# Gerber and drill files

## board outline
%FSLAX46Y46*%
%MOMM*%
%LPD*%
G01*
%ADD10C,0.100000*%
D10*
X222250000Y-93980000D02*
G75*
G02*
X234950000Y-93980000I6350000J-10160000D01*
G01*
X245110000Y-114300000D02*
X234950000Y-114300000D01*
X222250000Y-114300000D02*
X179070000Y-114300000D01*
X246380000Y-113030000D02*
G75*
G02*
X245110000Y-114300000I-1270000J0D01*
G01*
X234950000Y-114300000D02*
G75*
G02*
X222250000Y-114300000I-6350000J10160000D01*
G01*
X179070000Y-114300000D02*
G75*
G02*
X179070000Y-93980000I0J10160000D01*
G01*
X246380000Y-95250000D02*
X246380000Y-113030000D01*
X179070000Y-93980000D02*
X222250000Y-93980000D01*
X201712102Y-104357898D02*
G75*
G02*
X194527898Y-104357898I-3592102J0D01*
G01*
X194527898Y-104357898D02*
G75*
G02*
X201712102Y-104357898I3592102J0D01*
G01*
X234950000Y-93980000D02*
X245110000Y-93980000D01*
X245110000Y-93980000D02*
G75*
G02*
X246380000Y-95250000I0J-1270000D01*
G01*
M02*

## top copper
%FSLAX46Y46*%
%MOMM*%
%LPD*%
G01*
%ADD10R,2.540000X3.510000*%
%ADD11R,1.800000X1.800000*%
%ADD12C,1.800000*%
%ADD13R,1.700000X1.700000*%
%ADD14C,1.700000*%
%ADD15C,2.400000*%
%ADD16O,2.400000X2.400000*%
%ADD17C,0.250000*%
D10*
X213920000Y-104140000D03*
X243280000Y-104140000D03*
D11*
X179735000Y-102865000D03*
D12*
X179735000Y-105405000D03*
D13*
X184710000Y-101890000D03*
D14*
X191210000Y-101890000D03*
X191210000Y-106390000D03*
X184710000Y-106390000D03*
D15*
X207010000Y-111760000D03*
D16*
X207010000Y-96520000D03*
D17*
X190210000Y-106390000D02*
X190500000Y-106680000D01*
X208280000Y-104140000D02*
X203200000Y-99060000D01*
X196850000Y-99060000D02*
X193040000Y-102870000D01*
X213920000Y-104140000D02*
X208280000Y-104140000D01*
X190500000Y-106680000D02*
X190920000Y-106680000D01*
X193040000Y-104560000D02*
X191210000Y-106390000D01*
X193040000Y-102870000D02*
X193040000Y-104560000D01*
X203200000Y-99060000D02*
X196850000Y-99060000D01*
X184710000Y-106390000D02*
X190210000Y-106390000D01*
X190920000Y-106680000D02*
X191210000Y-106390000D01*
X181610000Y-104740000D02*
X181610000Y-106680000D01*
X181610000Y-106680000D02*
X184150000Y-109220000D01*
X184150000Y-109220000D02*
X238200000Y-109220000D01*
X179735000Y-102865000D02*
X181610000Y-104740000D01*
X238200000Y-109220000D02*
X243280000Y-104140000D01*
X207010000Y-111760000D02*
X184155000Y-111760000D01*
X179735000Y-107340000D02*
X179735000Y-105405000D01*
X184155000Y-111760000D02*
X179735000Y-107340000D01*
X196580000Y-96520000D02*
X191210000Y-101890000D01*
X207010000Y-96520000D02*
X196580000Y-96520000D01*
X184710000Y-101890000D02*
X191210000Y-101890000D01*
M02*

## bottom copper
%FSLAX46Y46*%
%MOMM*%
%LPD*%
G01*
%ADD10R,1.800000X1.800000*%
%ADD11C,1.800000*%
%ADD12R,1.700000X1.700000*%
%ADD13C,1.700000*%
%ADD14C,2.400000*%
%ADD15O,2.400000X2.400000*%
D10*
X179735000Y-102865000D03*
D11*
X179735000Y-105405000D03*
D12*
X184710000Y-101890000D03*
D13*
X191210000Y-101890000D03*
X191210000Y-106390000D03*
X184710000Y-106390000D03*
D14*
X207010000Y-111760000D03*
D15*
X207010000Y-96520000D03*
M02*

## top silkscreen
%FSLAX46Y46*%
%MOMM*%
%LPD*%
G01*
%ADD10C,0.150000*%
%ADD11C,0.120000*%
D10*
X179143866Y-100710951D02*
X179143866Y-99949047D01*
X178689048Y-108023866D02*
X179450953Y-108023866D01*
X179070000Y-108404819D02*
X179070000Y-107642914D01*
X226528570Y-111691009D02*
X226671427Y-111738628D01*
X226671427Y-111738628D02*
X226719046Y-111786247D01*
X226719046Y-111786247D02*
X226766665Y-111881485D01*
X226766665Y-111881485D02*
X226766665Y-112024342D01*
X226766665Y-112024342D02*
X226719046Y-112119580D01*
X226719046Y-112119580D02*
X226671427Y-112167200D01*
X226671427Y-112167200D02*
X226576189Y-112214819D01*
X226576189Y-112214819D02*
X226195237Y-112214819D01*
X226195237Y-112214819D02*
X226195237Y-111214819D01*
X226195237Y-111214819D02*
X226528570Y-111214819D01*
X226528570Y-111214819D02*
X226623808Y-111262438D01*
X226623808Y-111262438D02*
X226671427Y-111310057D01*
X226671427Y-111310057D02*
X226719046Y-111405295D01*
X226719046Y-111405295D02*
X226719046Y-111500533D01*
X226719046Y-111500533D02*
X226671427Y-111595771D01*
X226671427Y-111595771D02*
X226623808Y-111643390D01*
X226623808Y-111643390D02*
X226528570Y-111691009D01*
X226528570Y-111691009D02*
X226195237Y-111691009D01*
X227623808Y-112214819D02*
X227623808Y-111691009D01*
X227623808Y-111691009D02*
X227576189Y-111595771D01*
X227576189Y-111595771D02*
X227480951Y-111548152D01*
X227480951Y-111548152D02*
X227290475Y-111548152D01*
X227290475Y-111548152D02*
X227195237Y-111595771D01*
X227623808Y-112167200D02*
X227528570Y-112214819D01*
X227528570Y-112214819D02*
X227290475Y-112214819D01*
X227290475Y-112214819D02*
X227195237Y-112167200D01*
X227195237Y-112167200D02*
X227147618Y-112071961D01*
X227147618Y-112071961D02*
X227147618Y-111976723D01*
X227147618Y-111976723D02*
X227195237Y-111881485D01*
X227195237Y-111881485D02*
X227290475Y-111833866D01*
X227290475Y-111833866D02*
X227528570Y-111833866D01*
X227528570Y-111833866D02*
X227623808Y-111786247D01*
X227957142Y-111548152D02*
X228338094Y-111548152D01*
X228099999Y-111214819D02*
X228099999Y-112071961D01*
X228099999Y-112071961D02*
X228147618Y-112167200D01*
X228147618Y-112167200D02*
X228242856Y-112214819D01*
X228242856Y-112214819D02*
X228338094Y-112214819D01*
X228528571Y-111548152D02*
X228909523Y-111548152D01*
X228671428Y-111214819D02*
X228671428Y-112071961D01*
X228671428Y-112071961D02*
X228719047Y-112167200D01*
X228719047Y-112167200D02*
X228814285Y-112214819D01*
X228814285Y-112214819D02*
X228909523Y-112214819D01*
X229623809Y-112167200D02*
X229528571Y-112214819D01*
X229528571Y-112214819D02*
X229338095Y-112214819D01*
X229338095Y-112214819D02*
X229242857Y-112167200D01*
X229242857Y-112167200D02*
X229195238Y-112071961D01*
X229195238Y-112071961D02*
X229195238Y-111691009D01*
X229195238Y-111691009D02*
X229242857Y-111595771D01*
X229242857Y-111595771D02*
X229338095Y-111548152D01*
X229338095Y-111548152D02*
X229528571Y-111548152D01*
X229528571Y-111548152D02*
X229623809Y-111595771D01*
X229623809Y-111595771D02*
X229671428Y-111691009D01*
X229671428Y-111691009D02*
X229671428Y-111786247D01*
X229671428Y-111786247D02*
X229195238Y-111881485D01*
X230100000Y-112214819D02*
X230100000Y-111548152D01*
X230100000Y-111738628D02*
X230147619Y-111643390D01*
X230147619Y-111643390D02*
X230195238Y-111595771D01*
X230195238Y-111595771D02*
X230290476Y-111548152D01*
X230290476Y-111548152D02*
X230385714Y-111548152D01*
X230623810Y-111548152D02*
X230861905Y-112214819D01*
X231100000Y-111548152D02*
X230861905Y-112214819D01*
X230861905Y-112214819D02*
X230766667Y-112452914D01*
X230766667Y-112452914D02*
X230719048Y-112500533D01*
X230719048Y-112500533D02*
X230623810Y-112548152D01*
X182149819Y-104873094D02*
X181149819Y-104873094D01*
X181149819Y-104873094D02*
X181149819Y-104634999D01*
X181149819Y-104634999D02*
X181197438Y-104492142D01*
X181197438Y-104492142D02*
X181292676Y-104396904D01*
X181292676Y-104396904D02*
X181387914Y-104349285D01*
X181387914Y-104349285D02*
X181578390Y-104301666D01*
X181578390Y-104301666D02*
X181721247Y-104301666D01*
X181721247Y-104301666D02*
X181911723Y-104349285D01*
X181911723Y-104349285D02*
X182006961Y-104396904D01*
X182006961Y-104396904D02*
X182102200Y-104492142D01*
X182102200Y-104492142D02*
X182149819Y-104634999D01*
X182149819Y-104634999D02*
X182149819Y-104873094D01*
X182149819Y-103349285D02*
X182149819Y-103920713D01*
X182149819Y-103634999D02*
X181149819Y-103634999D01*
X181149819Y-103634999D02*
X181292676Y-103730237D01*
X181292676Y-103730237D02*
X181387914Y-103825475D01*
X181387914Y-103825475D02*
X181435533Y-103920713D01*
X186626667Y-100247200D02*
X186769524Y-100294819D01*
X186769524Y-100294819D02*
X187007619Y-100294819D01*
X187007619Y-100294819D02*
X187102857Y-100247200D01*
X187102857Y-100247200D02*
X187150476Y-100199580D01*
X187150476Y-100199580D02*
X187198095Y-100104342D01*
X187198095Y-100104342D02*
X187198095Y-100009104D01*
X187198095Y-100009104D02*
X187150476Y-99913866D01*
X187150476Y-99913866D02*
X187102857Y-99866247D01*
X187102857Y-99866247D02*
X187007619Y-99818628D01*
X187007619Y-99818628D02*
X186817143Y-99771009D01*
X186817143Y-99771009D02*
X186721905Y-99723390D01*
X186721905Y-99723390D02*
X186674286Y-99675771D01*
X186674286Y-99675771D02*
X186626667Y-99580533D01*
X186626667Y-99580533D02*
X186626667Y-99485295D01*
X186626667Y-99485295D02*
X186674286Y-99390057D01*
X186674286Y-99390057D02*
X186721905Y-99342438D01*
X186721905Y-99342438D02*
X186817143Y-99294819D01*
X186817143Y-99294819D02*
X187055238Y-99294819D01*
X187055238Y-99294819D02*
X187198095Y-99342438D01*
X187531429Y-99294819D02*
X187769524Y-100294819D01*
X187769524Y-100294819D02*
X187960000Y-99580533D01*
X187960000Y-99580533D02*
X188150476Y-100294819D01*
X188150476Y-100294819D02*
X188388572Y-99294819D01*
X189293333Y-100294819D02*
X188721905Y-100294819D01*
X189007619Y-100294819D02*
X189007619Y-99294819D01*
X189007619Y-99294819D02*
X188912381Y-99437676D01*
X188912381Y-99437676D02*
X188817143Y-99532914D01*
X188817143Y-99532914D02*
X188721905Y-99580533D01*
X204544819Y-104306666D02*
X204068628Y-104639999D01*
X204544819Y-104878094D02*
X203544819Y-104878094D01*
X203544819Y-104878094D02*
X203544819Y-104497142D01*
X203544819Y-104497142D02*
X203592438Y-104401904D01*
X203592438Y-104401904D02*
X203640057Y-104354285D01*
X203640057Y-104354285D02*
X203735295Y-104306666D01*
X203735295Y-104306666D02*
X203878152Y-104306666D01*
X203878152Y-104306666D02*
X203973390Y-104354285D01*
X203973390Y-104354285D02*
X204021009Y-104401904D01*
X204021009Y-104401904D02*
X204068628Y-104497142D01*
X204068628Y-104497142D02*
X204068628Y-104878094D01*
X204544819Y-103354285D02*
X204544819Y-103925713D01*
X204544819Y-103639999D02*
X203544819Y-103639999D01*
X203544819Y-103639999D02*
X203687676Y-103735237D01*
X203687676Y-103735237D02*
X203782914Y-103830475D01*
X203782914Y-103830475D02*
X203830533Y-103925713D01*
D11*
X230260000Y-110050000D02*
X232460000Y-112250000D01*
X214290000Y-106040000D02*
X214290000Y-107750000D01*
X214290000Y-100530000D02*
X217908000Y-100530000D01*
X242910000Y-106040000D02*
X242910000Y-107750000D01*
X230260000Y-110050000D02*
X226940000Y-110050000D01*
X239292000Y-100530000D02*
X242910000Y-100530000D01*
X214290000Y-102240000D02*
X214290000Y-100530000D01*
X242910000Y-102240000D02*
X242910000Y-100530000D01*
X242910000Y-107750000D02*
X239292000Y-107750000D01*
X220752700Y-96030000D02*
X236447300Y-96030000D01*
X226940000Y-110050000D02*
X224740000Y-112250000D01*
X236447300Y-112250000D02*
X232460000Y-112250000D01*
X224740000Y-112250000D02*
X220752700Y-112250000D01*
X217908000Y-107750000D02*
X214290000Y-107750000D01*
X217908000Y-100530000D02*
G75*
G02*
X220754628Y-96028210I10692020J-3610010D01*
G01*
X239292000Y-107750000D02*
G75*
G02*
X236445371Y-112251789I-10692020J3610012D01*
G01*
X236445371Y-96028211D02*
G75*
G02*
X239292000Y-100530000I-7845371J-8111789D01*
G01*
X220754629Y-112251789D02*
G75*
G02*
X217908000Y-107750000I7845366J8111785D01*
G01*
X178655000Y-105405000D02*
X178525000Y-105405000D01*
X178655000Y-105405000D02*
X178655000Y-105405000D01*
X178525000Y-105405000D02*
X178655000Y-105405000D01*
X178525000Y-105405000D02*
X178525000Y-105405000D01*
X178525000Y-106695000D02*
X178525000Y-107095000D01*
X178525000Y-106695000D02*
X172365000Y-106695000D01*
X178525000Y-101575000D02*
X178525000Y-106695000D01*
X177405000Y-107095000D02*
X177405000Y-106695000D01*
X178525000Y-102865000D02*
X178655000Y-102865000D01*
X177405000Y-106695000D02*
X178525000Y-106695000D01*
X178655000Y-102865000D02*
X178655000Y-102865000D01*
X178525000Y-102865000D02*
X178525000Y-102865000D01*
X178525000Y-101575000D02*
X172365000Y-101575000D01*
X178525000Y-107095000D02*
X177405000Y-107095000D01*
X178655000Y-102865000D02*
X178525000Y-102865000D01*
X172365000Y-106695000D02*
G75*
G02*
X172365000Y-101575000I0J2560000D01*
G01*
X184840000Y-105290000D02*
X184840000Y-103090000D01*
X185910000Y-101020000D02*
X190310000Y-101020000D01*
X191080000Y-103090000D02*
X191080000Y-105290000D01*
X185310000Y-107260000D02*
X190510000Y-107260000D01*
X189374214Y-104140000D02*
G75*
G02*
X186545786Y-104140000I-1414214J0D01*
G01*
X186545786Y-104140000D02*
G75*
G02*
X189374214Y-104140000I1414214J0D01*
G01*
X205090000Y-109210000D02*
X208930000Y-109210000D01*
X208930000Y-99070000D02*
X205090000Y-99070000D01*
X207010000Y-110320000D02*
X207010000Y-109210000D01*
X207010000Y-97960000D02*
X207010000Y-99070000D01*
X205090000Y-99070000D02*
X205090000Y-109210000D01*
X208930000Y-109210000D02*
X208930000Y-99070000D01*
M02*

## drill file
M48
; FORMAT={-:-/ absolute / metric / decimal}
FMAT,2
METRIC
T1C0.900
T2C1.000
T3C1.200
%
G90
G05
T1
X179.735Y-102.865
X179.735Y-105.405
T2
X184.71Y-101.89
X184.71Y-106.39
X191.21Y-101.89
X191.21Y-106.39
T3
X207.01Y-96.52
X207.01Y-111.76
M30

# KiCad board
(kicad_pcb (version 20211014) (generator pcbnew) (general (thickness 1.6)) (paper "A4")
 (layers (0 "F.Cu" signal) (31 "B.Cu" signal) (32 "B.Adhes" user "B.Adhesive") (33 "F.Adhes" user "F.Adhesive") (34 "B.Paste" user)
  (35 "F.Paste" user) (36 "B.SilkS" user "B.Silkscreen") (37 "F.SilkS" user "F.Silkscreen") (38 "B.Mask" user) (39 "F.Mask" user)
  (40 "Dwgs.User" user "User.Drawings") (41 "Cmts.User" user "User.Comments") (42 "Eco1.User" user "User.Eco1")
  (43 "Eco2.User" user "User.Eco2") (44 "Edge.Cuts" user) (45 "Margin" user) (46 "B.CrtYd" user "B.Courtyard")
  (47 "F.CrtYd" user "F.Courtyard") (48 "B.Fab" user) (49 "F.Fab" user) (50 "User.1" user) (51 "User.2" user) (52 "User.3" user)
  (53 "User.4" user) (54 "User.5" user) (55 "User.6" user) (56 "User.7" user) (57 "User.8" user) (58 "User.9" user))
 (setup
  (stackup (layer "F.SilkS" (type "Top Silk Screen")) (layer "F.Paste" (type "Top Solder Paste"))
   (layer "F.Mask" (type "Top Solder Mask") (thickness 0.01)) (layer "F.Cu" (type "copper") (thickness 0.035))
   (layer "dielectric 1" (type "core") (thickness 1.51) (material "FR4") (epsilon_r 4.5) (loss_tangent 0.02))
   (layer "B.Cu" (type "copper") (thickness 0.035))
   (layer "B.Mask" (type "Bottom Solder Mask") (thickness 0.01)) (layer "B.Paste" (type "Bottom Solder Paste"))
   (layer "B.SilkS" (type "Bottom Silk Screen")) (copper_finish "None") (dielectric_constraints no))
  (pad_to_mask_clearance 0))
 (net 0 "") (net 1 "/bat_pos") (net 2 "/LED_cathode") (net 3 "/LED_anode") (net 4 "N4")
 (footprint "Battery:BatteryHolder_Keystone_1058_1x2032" (layer "F.Cu") (at 228.6 104.14)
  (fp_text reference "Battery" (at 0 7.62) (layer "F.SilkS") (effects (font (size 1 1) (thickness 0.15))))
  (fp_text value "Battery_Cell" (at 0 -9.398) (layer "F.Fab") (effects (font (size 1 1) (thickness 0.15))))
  (fp_line (start 1.66 5.91) (end 3.86 8.11) (layer "F.SilkS") (width 0.12))
  (fp_line (start -14.31 1.9) (end -14.31 3.61) (layer "F.SilkS") (width 0.12))
  (fp_line (start -14.31 -3.61) (end -10.692 -3.61) (layer "F.SilkS") (width 0.12))
  (fp_line (start 14.31 1.9) (end 14.31 3.61) (layer "F.SilkS") (width 0.12))
  (fp_line (start 1.66 5.91) (end -1.66 5.91) (layer "F.SilkS") (width 0.12))
  (fp_line (start 10.692 -3.61) (end 14.31 -3.61) (layer "F.SilkS") (width 0.12))
  (fp_line (start -14.31 -1.9) (end -14.31 -3.61) (layer "F.SilkS") (width 0.12))
  (fp_line (start 14.31 -1.9) (end 14.31 -3.61) (layer "F.SilkS") (width 0.12))
  (fp_line (start 14.31 3.61) (end 10.692 3.61) (layer "F.SilkS") (width 0.12))
  (fp_line (start -7.8473 -8.11) (end 7.8473 -8.11) (layer "F.SilkS") (width 0.12))
  (fp_line (start -1.66 5.91) (end -3.86 8.11) (layer "F.SilkS") (width 0.12))
  (fp_line (start 7.8473 8.11) (end 3.86 8.11) (layer "F.SilkS") (width 0.12))
  (fp_line (start -3.86 8.11) (end -7.8473 8.11) (layer "F.SilkS") (width 0.12))
  (fp_line (start -10.692 3.61) (end -14.31 3.61) (layer "F.SilkS") (width 0.12))
  (fp_arc (start -10.692 -3.61) (mid -9.538084 -6.031244) (end -7.845371 -8.111789) (layer "F.SilkS") (width 0.12))
  (fp_arc (start 10.692 3.61) (mid 9.538084 6.031244) (end 7.845371 8.111789) (layer "F.SilkS") (width 0.12))
  (fp_arc (start 7.845371 -8.111789) (mid 9.538085 -6.031244) (end 10.692 -3.61) (layer "F.SilkS") (width 0.12))
  (fp_arc (start -7.845371 8.111789) (mid -9.538085 6.031244) (end -10.692 3.61) (layer "F.SilkS") (width 0.12))
  (pad "1" smd rect (at -14.68 0) (size 2.54 3.51) (layers "F.Cu" "F.Paste" "F.Mask") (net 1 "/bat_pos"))
  (pad "2" smd rect (at 14.68 0) (size 2.54 3.51) (layers "F.Cu" "F.Paste" "F.Mask") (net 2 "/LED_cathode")))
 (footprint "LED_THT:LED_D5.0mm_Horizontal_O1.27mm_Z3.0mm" (layer "F.Cu") (at 179.735 102.865 -90)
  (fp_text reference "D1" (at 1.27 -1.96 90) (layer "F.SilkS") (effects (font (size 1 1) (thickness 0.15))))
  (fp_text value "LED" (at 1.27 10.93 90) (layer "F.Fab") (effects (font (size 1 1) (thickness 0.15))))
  (fp_line (start 2.54 1.08) (end 2.54 1.21) (layer "F.SilkS") (width 0.12))
  (fp_line (start 2.54 1.08) (end 2.54 1.08) (layer "F.SilkS") (width 0.12))
  (fp_line (start 2.54 1.21) (end 2.54 1.08) (layer "F.SilkS") (width 0.12))
  (fp_line (start 2.54 1.21) (end 2.54 1.21) (layer "F.SilkS") (width 0.12))
  (fp_line (start 3.83 1.21) (end 4.23 1.21) (layer "F.SilkS") (width 0.12))
  (fp_line (start 3.83 1.21) (end 3.83 7.37) (layer "F.SilkS") (width 0.12))
  (fp_line (start -1.29 1.21) (end 3.83 1.21) (layer "F.SilkS") (width 0.12))
  (fp_line (start 4.23 2.33) (end 3.83 2.33) (layer "F.SilkS") (width 0.12))
  (fp_line (start 0 1.21) (end 0 1.08) (layer "F.SilkS") (width 0.12))
  (fp_line (start 3.83 2.33) (end 3.83 1.21) (layer "F.SilkS") (width 0.12))
  (fp_line (start 0 1.08) (end 0 1.08) (layer "F.SilkS") (width 0.12))
  (fp_line (start 0 1.21) (end 0 1.21) (layer "F.SilkS") (width 0.12))
  (fp_line (start -1.29 1.21) (end -1.29 7.37) (layer "F.SilkS") (width 0.12))
  (fp_line (start 4.23 1.21) (end 4.23 2.33) (layer "F.SilkS") (width 0.12))
  (fp_line (start 0 1.08) (end 0 1.21) (layer "F.SilkS") (width 0.12))
  (fp_arc (start 3.83 7.37) (mid 1.27 9.93) (end -1.29 7.37) (layer "F.SilkS") (width 0.12))
  (pad "1" thru_hole rect (at 0 0 270) (size 1.8 1.8) (drill 0.9) (layers *.Cu *.Mask) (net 2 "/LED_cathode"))
  (pad "2" thru_hole circle (at 2.54 0 270) (size 1.8 1.8) (drill 0.9) (layers *.Cu *.Mask) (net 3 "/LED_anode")))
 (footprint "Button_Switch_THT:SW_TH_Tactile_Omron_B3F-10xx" (layer "F.Cu") (at 184.71 101.89)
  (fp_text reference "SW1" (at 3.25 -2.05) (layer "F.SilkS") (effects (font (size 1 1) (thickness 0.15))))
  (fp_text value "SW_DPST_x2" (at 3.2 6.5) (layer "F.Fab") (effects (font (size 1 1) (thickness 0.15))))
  (fp_line (start 0.13 3.4) (end 0.13 1.2) (layer "F.SilkS") (width 0.12))
  (fp_line (start 1.2 -0.87) (end 5.6 -0.87) (layer "F.SilkS") (width 0.12))
  (fp_line (start 6.37 1.2) (end 6.37 3.4) (layer "F.SilkS") (width 0.12))
  (fp_line (start 0.6 5.37) (end 5.8 5.37) (layer "F.SilkS") (width 0.12))
  (fp_circle (center 3.25 2.25) (end 4.25 3.25) (layer "F.SilkS") (width 0.12) (fill none))
  (pad "1" thru_hole rect (at 0 0) (size 1.7 1.7) (drill 1) (layers *.Cu *.Mask) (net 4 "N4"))
  (pad "1" thru_hole circle (at 6.5 0) (size 1.7 1.7) (drill 1) (layers *.Cu *.Mask) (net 4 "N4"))
  (pad "2" thru_hole circle (at 6.5 4.5) (size 1.7 1.7) (drill 1) (layers *.Cu *.Mask) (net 1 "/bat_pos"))
  (pad "2" thru_hole circle (at 0 4.5) (size 1.7 1.7) (drill 1) (layers *.Cu *.Mask) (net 1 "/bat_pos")))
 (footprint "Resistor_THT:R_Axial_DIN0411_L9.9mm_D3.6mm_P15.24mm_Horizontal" (layer "F.Cu") (at 207.01 111.76 90)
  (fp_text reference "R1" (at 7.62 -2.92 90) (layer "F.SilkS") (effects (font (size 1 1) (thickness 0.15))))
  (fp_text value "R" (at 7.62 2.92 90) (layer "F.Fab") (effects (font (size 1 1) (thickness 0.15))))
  (fp_line (start 2.55 -1.92) (end 2.55 1.92) (layer "F.SilkS") (width 0.12))
  (fp_line (start 12.69 1.92) (end 12.69 -1.92) (layer "F.SilkS") (width 0.12))
  (fp_line (start 1.44 0) (end 2.55 0) (layer "F.SilkS") (width 0.12))
  (fp_line (start 13.8 0) (end 12.69 0) (layer "F.SilkS") (width 0.12))
  (fp_line (start 12.69 -1.92) (end 2.55 -1.92) (layer "F.SilkS") (width 0.12))
  (fp_line (start 2.55 1.92) (end 12.69 1.92) (layer "F.SilkS") (width 0.12))
  (pad "1" thru_hole circle (at 0 0 90) (size 2.4 2.4) (drill 1.2) (layers *.Cu *.Mask) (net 3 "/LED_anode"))
  (pad "2" thru_hole oval (at 15.24 0 90) (size 2.4 2.4) (drill 1.2) (layers *.Cu *.Mask) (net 4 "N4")))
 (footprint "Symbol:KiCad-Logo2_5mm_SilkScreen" (layer "B.Cu") (at 228.6 104.14 180)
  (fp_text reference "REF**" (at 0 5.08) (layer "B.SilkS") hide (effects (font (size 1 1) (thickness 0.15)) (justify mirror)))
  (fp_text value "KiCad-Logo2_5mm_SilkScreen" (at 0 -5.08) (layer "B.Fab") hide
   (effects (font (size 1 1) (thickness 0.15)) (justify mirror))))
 (gr_arc (start 222.25 93.98) (mid 228.6 92.158844) (end 234.95 93.98) (layer "Edge.Cuts") (width 0.1))
 (gr_line (start 245.11 114.3) (end 234.95 114.3) (layer "Edge.Cuts") (width 0.1))
 (gr_line (start 222.25 114.3) (end 179.07 114.3) (layer "Edge.Cuts") (width 0.1))
 (gr_arc (start 246.38 113.03) (mid 246.008026 113.928026) (end 245.11 114.3) (layer "Edge.Cuts") (width 0.1))
 (gr_arc (start 234.95 114.3) (mid 228.6 116.121156) (end 222.25 114.3) (layer "Edge.Cuts") (width 0.1))
 (gr_arc (start 179.07 114.3) (mid 168.91 104.14) (end 179.07 93.98) (layer "Edge.Cuts") (width 0.1))
 (gr_line (start 246.38 95.25) (end 246.38 113.03) (layer "Edge.Cuts") (width 0.1))
 (gr_line (start 179.07 93.98) (end 222.25 93.98) (layer "Edge.Cuts") (width 0.1))
 (gr_circle (center 198.12 104.357898) (end 200.66 106.897898) (layer "Edge.Cuts") (width 0.1) (fill none))
 (gr_line (start 234.95 93.98) (end 245.11 93.98) (layer "Edge.Cuts") (width 0.1))
 (gr_arc (start 245.11 93.98) (mid 246.008026 94.351974) (end 246.38 95.25) (layer "Edge.Cuts") (width 0.1))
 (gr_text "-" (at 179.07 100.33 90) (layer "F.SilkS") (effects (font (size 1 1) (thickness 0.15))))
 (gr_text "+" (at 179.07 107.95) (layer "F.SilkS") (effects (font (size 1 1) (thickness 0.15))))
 (segment (start 190.21 106.39) (end 190.5 106.68) (width 0.25) (layer "F.Cu") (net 1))
 (segment (start 208.28 104.14) (end 203.2 99.06) (width 0.25) (layer "F.Cu") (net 1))
 (segment (start 196.85 99.06) (end 193.04 102.87) (width 0.25) (layer "F.Cu") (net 1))
 (segment (start 213.92 104.14) (end 208.28 104.14) (width 0.25) (layer "F.Cu") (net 1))
 (segment (start 190.5 106.68) (end 190.92 106.68) (width 0.25) (layer "F.Cu") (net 1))
 (segment (start 193.04 104.56) (end 191.21 106.39) (width 0.25) (layer "F.Cu") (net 1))
 (segment (start 193.04 102.87) (end 193.04 104.56) (width 0.25) (layer "F.Cu") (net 1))
 (segment (start 203.2 99.06) (end 196.85 99.06) (width 0.25) (layer "F.Cu") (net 1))
 (segment (start 184.71 106.39) (end 190.21 106.39) (width 0.25) (layer "F.Cu") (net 1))
 (segment (start 190.92 106.68) (end 191.21 106.39) (width 0.25) (layer "F.Cu") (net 1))
 (segment (start 181.61 104.74) (end 181.61 106.68) (width 0.25) (layer "F.Cu") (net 2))
 (segment (start 181.61 106.68) (end 184.15 109.22) (width 0.25) (layer "F.Cu") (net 2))
 (segment (start 184.15 109.22) (end 238.2 109.22) (width 0.25) (layer "F.Cu") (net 2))
 (segment (start 179.735 102.865) (end 181.61 104.74) (width 0.25) (layer "F.Cu") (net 2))
 (segment (start 238.2 109.22) (end 243.28 104.14) (width 0.25) (layer "F.Cu") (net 2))
 (segment (start 207.01 111.76) (end 184.155 111.76) (width 0.25) (layer "F.Cu") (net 3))
 (segment (start 179.735 107.34) (end 179.735 105.405) (width 0.25) (layer "F.Cu") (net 3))
 (segment (start 184.155 111.76) (end 179.735 107.34) (width 0.25) (layer "F.Cu") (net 3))
 (segment (start 196.58 96.52) (end 191.21 101.89) (width 0.25) (layer "F.Cu") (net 4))
 (segment (start 207.01 96.52) (end 196.58 96.52) (width 0.25) (layer "F.Cu") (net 4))
 (segment (start 184.71 101.89) (end 191.21 101.89) (width 0.25) (layer "F.Cu") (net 4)))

